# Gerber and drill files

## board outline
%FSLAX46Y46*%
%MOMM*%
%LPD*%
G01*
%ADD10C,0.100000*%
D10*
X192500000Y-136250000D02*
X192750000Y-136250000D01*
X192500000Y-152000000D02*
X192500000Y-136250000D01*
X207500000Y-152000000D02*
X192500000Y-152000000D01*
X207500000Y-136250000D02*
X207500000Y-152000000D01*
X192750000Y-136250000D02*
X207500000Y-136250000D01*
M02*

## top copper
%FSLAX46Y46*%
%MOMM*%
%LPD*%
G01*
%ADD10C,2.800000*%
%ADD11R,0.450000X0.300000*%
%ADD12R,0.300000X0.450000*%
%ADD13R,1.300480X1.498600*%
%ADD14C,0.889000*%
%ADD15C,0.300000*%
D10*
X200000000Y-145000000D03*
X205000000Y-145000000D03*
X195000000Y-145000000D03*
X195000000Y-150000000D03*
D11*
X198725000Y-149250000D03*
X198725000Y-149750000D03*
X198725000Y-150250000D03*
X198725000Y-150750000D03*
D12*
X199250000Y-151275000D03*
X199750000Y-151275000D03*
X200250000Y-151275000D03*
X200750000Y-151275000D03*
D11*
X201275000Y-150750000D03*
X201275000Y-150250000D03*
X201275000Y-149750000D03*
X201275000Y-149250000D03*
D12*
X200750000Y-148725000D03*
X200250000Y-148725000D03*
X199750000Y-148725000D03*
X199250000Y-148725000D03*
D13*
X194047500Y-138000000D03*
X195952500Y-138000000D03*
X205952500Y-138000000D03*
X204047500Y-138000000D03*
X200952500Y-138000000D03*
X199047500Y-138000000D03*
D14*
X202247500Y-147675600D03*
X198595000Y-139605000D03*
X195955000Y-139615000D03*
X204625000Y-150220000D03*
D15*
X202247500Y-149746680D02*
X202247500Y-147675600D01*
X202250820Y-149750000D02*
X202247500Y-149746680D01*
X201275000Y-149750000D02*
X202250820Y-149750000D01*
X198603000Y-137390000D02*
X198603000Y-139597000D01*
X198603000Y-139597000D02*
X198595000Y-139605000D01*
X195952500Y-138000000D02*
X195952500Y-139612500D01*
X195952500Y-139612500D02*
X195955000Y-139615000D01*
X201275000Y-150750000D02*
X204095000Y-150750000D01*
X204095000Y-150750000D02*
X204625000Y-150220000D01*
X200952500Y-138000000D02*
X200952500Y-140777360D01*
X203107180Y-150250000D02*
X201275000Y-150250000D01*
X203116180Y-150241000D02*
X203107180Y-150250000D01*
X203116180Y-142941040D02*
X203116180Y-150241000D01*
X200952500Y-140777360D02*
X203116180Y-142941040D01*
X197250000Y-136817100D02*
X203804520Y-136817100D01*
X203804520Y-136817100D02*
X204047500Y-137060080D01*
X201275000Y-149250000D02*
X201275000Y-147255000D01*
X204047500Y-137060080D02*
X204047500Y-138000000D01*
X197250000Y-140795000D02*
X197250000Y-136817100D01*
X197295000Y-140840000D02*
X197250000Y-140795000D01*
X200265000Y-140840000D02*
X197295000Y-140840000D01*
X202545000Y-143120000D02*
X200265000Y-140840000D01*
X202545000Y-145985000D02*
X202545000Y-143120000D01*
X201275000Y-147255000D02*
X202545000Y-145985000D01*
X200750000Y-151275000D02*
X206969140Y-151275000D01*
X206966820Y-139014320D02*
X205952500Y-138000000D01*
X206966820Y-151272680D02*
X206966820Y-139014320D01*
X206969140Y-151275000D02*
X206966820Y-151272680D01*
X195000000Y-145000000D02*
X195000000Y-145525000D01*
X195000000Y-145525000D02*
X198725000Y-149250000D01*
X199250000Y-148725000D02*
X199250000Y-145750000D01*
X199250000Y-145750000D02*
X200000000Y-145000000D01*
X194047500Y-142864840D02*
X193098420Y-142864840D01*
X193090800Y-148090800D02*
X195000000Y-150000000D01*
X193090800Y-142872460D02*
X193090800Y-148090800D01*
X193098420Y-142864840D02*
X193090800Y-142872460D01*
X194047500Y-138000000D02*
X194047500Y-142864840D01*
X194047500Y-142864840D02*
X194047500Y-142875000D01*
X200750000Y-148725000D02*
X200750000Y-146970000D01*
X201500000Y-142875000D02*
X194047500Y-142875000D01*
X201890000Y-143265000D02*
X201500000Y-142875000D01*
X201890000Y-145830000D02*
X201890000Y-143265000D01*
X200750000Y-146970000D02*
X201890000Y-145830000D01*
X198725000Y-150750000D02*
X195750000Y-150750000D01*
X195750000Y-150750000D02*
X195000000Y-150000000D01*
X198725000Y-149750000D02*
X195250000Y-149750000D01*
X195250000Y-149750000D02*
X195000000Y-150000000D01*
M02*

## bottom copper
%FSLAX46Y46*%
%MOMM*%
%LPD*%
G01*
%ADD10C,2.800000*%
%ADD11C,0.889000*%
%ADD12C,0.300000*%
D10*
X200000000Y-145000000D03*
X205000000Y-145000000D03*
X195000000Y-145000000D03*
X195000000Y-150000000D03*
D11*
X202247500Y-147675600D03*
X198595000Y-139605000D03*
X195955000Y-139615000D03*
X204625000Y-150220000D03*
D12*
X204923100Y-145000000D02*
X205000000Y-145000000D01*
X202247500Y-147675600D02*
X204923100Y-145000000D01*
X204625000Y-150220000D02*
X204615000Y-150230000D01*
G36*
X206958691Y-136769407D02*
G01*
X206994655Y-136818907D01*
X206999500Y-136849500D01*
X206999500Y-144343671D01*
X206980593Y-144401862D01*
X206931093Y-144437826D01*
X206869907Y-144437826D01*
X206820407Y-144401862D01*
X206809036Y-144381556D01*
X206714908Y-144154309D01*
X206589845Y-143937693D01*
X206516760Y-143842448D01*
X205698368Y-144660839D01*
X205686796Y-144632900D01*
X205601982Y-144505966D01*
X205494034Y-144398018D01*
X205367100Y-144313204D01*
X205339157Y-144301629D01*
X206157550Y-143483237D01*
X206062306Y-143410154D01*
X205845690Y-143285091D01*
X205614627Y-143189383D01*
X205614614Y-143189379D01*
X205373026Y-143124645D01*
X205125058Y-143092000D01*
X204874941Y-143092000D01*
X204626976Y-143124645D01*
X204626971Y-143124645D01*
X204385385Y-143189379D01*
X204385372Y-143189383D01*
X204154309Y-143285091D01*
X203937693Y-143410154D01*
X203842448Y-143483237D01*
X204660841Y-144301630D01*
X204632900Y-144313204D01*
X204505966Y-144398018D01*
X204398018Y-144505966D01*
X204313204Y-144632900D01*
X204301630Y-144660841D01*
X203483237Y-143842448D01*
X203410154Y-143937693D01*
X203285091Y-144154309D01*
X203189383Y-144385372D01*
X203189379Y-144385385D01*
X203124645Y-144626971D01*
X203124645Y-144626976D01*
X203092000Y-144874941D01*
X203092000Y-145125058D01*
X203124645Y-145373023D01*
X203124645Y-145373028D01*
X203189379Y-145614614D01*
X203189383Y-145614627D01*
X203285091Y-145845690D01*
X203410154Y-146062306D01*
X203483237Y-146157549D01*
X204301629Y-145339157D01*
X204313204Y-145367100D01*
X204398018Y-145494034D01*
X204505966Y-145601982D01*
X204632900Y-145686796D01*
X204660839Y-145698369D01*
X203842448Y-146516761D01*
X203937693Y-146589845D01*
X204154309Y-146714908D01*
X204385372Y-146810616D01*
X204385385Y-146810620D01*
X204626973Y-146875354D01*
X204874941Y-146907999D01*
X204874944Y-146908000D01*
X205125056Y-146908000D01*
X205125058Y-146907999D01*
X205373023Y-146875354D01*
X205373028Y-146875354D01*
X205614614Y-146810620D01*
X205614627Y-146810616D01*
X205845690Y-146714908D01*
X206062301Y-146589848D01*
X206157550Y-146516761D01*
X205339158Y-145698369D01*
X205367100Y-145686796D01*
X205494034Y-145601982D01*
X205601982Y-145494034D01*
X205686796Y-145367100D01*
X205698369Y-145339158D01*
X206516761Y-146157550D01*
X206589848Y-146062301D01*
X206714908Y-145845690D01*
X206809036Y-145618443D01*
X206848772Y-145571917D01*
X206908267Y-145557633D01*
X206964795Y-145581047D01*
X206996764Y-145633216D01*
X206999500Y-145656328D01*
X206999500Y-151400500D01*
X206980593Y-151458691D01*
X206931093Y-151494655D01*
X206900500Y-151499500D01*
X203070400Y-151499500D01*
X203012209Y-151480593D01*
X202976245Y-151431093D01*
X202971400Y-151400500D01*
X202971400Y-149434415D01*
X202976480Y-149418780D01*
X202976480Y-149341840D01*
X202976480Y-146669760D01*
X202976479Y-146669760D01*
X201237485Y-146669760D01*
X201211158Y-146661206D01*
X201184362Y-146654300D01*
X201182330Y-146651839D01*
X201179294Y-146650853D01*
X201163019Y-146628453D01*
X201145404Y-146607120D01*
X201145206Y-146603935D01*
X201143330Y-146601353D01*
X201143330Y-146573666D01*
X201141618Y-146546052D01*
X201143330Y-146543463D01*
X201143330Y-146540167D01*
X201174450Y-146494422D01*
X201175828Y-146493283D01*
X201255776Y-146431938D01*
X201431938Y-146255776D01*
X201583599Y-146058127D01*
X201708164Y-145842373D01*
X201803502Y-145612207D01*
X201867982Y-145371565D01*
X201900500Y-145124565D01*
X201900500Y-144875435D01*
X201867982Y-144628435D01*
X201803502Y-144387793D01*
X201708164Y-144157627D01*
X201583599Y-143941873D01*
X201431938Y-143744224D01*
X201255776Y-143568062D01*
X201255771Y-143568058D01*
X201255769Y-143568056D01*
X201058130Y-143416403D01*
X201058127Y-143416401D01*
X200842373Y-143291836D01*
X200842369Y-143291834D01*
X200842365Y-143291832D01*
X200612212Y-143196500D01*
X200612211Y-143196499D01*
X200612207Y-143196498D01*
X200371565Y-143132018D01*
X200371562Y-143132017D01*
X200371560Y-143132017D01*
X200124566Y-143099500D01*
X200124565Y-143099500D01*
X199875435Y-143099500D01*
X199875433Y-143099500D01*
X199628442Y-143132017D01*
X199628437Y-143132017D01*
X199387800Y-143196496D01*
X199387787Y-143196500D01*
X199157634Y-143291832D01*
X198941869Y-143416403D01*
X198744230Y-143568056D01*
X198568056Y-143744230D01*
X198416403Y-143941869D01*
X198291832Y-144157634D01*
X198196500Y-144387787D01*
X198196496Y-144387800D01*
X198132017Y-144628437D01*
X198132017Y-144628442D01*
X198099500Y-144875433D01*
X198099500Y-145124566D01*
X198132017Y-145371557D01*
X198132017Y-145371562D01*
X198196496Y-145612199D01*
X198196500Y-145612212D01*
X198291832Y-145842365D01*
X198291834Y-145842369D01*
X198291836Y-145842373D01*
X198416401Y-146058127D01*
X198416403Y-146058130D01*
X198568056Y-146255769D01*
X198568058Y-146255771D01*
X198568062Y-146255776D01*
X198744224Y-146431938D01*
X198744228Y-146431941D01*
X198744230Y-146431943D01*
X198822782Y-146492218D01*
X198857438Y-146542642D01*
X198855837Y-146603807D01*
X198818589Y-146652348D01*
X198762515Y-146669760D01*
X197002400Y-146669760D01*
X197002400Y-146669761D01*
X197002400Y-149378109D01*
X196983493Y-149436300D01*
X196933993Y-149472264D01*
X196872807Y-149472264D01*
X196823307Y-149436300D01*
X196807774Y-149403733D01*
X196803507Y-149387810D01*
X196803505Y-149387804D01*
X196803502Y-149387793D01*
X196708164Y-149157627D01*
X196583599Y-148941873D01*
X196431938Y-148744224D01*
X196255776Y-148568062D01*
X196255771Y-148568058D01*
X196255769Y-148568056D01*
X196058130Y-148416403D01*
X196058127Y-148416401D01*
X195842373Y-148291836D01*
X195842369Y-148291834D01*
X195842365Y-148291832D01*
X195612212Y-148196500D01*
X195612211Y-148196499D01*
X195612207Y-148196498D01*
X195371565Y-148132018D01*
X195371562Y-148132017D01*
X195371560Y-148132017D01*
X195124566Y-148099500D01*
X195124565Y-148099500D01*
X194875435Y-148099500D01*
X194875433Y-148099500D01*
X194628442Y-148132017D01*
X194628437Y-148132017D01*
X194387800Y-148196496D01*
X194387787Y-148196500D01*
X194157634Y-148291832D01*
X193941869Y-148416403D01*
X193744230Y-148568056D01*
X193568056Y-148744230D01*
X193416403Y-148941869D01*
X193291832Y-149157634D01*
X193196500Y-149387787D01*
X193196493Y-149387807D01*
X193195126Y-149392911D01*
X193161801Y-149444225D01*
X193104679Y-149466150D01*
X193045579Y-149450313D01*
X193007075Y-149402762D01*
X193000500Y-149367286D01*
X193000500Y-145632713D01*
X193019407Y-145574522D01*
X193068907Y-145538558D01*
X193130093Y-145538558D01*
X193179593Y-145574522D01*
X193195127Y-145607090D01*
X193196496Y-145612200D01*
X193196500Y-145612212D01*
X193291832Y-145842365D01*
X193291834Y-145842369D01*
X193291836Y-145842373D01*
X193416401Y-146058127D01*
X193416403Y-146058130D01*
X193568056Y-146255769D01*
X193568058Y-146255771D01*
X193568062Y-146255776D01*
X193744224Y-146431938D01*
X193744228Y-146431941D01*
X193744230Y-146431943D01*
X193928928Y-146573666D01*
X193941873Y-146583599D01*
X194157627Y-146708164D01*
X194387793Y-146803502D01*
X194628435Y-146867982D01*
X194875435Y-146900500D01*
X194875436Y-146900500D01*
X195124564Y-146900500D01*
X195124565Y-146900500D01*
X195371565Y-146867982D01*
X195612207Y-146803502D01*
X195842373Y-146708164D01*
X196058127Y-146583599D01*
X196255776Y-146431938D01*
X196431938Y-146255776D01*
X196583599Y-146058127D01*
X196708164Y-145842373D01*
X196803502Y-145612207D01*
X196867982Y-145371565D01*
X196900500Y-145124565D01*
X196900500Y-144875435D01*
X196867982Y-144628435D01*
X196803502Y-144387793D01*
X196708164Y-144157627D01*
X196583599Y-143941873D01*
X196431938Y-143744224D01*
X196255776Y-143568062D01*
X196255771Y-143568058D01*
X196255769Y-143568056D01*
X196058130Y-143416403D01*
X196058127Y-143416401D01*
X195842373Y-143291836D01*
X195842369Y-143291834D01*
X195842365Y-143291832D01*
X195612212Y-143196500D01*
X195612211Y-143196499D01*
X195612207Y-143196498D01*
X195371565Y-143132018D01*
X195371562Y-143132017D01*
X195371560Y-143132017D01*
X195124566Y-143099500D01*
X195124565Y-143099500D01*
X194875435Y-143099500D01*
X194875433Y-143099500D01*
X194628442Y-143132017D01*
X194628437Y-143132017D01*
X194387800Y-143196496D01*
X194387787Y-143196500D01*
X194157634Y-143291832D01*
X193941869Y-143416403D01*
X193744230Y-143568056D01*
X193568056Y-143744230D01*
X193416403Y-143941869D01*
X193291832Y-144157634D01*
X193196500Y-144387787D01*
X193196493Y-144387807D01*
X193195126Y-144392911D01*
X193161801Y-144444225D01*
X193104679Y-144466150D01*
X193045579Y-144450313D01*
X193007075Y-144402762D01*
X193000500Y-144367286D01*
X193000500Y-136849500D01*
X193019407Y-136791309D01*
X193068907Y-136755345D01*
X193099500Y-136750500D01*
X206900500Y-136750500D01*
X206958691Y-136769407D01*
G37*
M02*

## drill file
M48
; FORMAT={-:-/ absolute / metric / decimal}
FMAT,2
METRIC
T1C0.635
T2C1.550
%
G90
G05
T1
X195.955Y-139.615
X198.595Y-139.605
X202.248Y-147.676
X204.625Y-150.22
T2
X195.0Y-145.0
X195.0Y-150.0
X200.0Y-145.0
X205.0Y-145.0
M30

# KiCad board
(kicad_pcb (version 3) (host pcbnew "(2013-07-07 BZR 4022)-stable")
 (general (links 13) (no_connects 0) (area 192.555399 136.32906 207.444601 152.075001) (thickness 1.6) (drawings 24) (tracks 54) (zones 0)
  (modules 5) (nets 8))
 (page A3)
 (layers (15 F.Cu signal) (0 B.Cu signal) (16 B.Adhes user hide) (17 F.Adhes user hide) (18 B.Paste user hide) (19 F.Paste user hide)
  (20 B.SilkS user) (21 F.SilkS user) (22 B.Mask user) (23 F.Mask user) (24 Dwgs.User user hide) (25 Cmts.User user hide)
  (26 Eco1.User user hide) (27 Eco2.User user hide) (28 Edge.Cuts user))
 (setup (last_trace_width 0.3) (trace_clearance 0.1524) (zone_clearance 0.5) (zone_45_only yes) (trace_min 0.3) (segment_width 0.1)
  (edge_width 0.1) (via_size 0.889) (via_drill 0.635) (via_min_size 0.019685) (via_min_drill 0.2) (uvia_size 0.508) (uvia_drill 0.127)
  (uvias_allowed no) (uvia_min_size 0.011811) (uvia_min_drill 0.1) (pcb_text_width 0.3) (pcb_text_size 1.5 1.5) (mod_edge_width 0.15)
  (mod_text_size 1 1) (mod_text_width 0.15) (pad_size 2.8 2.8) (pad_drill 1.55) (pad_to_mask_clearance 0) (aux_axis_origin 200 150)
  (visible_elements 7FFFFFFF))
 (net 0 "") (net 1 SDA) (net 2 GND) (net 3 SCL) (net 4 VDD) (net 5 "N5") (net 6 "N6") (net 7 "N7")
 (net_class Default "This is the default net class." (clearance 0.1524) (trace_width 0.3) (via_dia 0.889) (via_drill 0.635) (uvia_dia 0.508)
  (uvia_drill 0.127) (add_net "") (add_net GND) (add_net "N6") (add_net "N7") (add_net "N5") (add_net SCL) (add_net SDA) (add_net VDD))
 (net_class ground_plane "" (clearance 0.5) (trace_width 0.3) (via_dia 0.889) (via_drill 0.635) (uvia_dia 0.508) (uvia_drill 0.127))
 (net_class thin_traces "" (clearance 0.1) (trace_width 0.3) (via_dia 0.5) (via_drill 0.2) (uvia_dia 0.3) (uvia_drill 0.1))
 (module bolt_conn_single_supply (layer F.Cu) (at 200 150)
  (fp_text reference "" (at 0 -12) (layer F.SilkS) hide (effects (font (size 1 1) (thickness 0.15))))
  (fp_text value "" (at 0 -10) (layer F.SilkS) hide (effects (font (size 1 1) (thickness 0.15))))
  (pad 4 thru_hole circle (at 0 -5) (size 2.8 2.8) (drill 1.55) (layers *.Cu F.SilkS F.Mask) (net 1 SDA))
  (pad 2 thru_hole circle (at 5 -5) (size 2.8 2.8) (drill 1.55) (layers *.Cu F.SilkS F.Mask) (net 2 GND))
  (pad 3 thru_hole circle (at -5 -5) (size 2.8 2.8) (drill 1.55) (layers *.Cu F.SilkS F.Mask) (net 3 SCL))
  (pad 1 thru_hole circle (at -5 0) (size 2.8 2.8) (drill 1.55) (layers *.Cu F.SilkS F.Mask) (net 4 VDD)))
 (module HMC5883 (layer F.Cu) (at 200 150)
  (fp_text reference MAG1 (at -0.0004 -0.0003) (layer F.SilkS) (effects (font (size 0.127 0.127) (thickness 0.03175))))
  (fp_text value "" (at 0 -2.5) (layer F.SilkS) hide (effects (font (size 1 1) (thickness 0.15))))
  (pad 1 smd rect (at -1.275 -0.75) (size 0.45 0.3) (layers F.Cu F.Paste F.Mask) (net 3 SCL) (clearance 0.05) (zone_connect 1))
  (pad 2 smd rect (at -1.275 -0.25) (size 0.45 0.3) (layers F.Cu F.Paste F.Mask) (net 4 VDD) (clearance 0.05))
  (pad 3 smd rect (at -1.275 0.25) (size 0.45 0.3) (layers F.Cu F.Paste F.Mask) (clearance 0.05))
  (pad 4 smd rect (at -1.275 0.75) (size 0.45 0.3) (layers F.Cu F.Paste F.Mask) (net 4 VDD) (clearance 0.05))
  (pad 5 smd rect (at -0.75 1.275 90) (size 0.45 0.3) (layers F.Cu F.Paste F.Mask) (clearance 0.05))
  (pad 6 smd rect (at -0.25 1.275 90) (size 0.45 0.3) (layers F.Cu F.Paste F.Mask) (clearance 0.05))
  (pad 7 smd rect (at 0.25 1.275 90) (size 0.45 0.3) (layers F.Cu F.Paste F.Mask) (clearance 0.05))
  (pad 8 smd rect (at 0.75 1.275 90) (size 0.45 0.3) (layers F.Cu F.Paste F.Mask) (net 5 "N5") (clearance 0.05))
  (pad 9 smd rect (at 1.275 0.75) (size 0.45 0.3) (layers F.Cu F.Paste F.Mask) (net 2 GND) (clearance 0.05))
  (pad 10 smd rect (at 1.275 0.25) (size 0.45 0.3) (layers F.Cu F.Paste F.Mask) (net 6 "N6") (clearance 0.05))
  (pad 11 smd rect (at 1.275 -0.25) (size 0.45 0.3) (layers F.Cu F.Paste F.Mask) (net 2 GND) (clearance 0.05))
  (pad 12 smd rect (at 1.275 -0.75) (size 0.45 0.3) (layers F.Cu F.Paste F.Mask) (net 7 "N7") (clearance 0.05))
  (pad 13 smd rect (at 0.75 -1.275 90) (size 0.45 0.3) (layers F.Cu F.Paste F.Mask) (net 4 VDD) (clearance 0.05))
  (pad 14 smd rect (at 0.25 -1.275 90) (size 0.45 0.3) (layers F.Cu F.Paste F.Mask) (clearance 0.05))
  (pad 15 smd rect (at -0.25 -1.275 90) (size 0.45 0.3) (layers F.Cu F.Paste F.Mask) (clearance 0.05))
  (pad 16 smd rect (at -0.75 -1.275 90) (size 0.45 0.3) (layers F.Cu F.Paste F.Mask) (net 1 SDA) (clearance 0.05)))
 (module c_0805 (layer F.Cu) (at 195 138 180)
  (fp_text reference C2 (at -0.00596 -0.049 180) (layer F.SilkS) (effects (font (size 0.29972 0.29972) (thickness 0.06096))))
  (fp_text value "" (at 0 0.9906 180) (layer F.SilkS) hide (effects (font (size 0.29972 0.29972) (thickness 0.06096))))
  (pad 1 smd rect (at 0.9525 0 180) (size 1.30048 1.4986) (layers F.Cu F.Paste F.Mask) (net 4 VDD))
  (pad 2 smd rect (at -0.9525 0 180) (size 1.30048 1.4986) (layers F.Cu F.Paste F.Mask) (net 2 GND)))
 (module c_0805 (layer F.Cu) (at 205 138)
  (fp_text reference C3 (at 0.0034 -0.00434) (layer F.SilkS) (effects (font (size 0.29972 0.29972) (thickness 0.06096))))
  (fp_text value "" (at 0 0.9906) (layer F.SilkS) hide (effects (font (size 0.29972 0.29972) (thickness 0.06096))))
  (pad 1 smd rect (at 0.9525 0) (size 1.30048 1.4986) (layers F.Cu F.Paste F.Mask) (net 5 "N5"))
  (pad 2 smd rect (at -0.9525 0) (size 1.30048 1.4986) (layers F.Cu F.Paste F.Mask) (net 7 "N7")))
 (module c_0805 (layer F.Cu) (at 200 138)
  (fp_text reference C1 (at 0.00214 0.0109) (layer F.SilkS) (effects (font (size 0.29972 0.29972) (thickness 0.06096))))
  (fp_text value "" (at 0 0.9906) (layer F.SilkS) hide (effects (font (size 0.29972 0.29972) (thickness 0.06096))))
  (pad 1 smd rect (at 0.9525 0) (size 1.30048 1.4986) (layers F.Cu F.Paste F.Mask) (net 6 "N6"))
  (pad 2 smd rect (at -0.9525 0) (size 1.30048 1.4986) (layers F.Cu F.Paste F.Mask) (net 2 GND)))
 (gr_line (start 192.5 136.25) (end 192.75 136.25) (angle 90) (layer Edge.Cuts) (width 0.1))
 (gr_line (start 192.5 152) (end 192.5 136.25) (angle 90) (layer Edge.Cuts) (width 0.1))
 (gr_line (start 207.5 152) (end 192.5 152) (angle 90) (layer Edge.Cuts) (width 0.1))
 (gr_line (start 207.5 136.25) (end 207.5 152) (angle 90) (layer Edge.Cuts) (width 0.1))
 (gr_line (start 192.75 136.25) (end 207.5 136.25) (angle 90) (layer Edge.Cuts) (width 0.1))
 (segment (start 204.9231 145) (end 205 145) (width 0.3) (layer B.Cu) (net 2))
 (segment (start 202.2475 147.6756) (end 204.9231 145) (width 0.3) (layer B.Cu) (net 2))
 (via (at 202.2475 147.6756) (size 0.889) (layers F.Cu B.Cu) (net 2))
 (segment (start 202.2475 149.74668) (end 202.2475 147.6756) (width 0.3) (layer F.Cu) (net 2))
 (segment (start 202.25082 149.75) (end 202.2475 149.74668) (width 0.3) (layer F.Cu) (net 2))
 (segment (start 201.275 149.75) (end 202.25082 149.75) (width 0.3) (layer F.Cu) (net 2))
 (segment (start 198.603 137.39) (end 198.603 139.597) (width 0.3) (layer F.Cu) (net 2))
 (via (at 198.595 139.605) (size 0.889) (layers F.Cu B.Cu) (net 2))
 (segment (start 198.603 139.597) (end 198.595 139.605) (width 0.3) (layer F.Cu) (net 2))
 (segment (start 195.9525 138) (end 195.9525 139.6125) (width 0.3) (layer F.Cu) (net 2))
 (via (at 195.955 139.615) (size 0.889) (layers F.Cu B.Cu) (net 2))
 (segment (start 195.9525 139.6125) (end 195.955 139.615) (width 0.3) (layer F.Cu) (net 2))
 (segment (start 201.275 150.75) (end 204.095 150.75) (width 0.3) (layer F.Cu) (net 2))
 (segment (start 204.625 150.22) (end 204.615 150.23) (width 0.3) (layer B.Cu) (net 2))
 (via (at 204.625 150.22) (size 0.889) (layers F.Cu B.Cu) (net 2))
 (segment (start 204.095 150.75) (end 204.625 150.22) (width 0.3) (layer F.Cu) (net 2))
 (segment (start 200.9525 138) (end 200.9525 140.77736) (width 0.3) (layer F.Cu) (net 6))
 (segment (start 203.10718 150.25) (end 201.275 150.25) (width 0.3) (layer F.Cu) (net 6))
 (segment (start 203.11618 150.241) (end 203.10718 150.25) (width 0.3) (layer F.Cu) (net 6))
 (segment (start 203.11618 142.94104) (end 203.11618 150.241) (width 0.3) (layer F.Cu) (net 6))
 (segment (start 200.9525 140.77736) (end 203.11618 142.94104) (width 0.3) (layer F.Cu) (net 6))
 (segment (start 197.25 136.8171) (end 203.80452 136.8171) (width 0.3) (layer F.Cu) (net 7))
 (segment (start 203.80452 136.8171) (end 204.0475 137.06008) (width 0.3) (layer F.Cu) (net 7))
 (segment (start 201.275 149.25) (end 201.275 147.255) (width 0.3) (layer F.Cu) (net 7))
 (segment (start 204.0475 137.06008) (end 204.0475 138) (width 0.3) (layer F.Cu) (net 7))
 (segment (start 197.25 140.795) (end 197.25 136.8171) (width 0.3) (layer F.Cu) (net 7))
 (segment (start 197.295 140.84) (end 197.25 140.795) (width 0.3) (layer F.Cu) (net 7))
 (segment (start 200.265 140.84) (end 197.295 140.84) (width 0.3) (layer F.Cu) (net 7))
 (segment (start 202.545 143.12) (end 200.265 140.84) (width 0.3) (layer F.Cu) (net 7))
 (segment (start 202.545 145.985) (end 202.545 143.12) (width 0.3) (layer F.Cu) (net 7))
 (segment (start 201.275 147.255) (end 202.545 145.985) (width 0.3) (layer F.Cu) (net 7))
 (segment (start 200.75 151.275) (end 206.96914 151.275) (width 0.3) (layer F.Cu) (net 5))
 (segment (start 206.96682 139.01432) (end 205.9525 138) (width 0.3) (layer F.Cu) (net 5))
 (segment (start 206.96682 151.27268) (end 206.96682 139.01432) (width 0.3) (layer F.Cu) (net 5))
 (segment (start 206.96914 151.275) (end 206.96682 151.27268) (width 0.3) (layer F.Cu) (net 5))
 (segment (start 195 145) (end 195 145.525) (width 0.3) (layer F.Cu) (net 3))
 (segment (start 195 145.525) (end 198.725 149.25) (width 0.3) (layer F.Cu) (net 3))
 (segment (start 199.25 148.725) (end 199.25 145.75) (width 0.3) (layer F.Cu) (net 1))
 (segment (start 199.25 145.75) (end 200 145) (width 0.3) (layer F.Cu) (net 1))
 (segment (start 194.0475 142.86484) (end 193.09842 142.86484) (width 0.3) (layer F.Cu) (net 4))
 (segment (start 193.0908 148.0908) (end 195 150) (width 0.3) (layer F.Cu) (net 4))
 (segment (start 193.0908 142.87246) (end 193.0908 148.0908) (width 0.3) (layer F.Cu) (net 4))
 (segment (start 193.09842 142.86484) (end 193.0908 142.87246) (width 0.3) (layer F.Cu) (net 4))
 (segment (start 194.0475 138) (end 194.0475 142.86484) (width 0.3) (layer F.Cu) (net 4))
 (segment (start 194.0475 142.86484) (end 194.0475 142.875) (width 0.3) (layer F.Cu) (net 4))
 (segment (start 200.75 148.725) (end 200.75 146.97) (width 0.3) (layer F.Cu) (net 4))
 (segment (start 201.5 142.875) (end 194.0475 142.875) (width 0.3) (layer F.Cu) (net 4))
 (segment (start 201.89 143.265) (end 201.5 142.875) (width 0.3) (layer F.Cu) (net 4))
 (segment (start 201.89 145.83) (end 201.89 143.265) (width 0.3) (layer F.Cu) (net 4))
 (segment (start 200.75 146.97) (end 201.89 145.83) (width 0.3) (layer F.Cu) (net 4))
 (segment (start 198.725 150.75) (end 195.75 150.75) (width 0.3) (layer F.Cu) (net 4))
 (segment (start 195.75 150.75) (end 195 150) (width 0.3) (layer F.Cu) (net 4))
 (segment (start 198.725 149.75) (end 195.25 149.75) (width 0.3) (layer F.Cu) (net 4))
 (segment (start 195.25 149.75) (end 195 150) (width 0.3) (layer F.Cu) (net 4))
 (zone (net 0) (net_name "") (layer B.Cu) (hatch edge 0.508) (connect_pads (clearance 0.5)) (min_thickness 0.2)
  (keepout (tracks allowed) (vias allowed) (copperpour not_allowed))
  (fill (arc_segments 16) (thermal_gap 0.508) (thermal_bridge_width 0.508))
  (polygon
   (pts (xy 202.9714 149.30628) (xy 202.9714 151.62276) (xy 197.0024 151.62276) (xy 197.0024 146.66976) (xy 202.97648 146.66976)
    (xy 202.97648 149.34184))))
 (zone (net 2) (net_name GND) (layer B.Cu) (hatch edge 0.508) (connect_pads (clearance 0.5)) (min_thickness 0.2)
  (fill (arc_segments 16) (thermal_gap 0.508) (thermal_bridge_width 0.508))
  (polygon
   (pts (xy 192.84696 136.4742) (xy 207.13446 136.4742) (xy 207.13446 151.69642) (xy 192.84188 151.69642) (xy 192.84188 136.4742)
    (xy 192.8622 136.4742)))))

